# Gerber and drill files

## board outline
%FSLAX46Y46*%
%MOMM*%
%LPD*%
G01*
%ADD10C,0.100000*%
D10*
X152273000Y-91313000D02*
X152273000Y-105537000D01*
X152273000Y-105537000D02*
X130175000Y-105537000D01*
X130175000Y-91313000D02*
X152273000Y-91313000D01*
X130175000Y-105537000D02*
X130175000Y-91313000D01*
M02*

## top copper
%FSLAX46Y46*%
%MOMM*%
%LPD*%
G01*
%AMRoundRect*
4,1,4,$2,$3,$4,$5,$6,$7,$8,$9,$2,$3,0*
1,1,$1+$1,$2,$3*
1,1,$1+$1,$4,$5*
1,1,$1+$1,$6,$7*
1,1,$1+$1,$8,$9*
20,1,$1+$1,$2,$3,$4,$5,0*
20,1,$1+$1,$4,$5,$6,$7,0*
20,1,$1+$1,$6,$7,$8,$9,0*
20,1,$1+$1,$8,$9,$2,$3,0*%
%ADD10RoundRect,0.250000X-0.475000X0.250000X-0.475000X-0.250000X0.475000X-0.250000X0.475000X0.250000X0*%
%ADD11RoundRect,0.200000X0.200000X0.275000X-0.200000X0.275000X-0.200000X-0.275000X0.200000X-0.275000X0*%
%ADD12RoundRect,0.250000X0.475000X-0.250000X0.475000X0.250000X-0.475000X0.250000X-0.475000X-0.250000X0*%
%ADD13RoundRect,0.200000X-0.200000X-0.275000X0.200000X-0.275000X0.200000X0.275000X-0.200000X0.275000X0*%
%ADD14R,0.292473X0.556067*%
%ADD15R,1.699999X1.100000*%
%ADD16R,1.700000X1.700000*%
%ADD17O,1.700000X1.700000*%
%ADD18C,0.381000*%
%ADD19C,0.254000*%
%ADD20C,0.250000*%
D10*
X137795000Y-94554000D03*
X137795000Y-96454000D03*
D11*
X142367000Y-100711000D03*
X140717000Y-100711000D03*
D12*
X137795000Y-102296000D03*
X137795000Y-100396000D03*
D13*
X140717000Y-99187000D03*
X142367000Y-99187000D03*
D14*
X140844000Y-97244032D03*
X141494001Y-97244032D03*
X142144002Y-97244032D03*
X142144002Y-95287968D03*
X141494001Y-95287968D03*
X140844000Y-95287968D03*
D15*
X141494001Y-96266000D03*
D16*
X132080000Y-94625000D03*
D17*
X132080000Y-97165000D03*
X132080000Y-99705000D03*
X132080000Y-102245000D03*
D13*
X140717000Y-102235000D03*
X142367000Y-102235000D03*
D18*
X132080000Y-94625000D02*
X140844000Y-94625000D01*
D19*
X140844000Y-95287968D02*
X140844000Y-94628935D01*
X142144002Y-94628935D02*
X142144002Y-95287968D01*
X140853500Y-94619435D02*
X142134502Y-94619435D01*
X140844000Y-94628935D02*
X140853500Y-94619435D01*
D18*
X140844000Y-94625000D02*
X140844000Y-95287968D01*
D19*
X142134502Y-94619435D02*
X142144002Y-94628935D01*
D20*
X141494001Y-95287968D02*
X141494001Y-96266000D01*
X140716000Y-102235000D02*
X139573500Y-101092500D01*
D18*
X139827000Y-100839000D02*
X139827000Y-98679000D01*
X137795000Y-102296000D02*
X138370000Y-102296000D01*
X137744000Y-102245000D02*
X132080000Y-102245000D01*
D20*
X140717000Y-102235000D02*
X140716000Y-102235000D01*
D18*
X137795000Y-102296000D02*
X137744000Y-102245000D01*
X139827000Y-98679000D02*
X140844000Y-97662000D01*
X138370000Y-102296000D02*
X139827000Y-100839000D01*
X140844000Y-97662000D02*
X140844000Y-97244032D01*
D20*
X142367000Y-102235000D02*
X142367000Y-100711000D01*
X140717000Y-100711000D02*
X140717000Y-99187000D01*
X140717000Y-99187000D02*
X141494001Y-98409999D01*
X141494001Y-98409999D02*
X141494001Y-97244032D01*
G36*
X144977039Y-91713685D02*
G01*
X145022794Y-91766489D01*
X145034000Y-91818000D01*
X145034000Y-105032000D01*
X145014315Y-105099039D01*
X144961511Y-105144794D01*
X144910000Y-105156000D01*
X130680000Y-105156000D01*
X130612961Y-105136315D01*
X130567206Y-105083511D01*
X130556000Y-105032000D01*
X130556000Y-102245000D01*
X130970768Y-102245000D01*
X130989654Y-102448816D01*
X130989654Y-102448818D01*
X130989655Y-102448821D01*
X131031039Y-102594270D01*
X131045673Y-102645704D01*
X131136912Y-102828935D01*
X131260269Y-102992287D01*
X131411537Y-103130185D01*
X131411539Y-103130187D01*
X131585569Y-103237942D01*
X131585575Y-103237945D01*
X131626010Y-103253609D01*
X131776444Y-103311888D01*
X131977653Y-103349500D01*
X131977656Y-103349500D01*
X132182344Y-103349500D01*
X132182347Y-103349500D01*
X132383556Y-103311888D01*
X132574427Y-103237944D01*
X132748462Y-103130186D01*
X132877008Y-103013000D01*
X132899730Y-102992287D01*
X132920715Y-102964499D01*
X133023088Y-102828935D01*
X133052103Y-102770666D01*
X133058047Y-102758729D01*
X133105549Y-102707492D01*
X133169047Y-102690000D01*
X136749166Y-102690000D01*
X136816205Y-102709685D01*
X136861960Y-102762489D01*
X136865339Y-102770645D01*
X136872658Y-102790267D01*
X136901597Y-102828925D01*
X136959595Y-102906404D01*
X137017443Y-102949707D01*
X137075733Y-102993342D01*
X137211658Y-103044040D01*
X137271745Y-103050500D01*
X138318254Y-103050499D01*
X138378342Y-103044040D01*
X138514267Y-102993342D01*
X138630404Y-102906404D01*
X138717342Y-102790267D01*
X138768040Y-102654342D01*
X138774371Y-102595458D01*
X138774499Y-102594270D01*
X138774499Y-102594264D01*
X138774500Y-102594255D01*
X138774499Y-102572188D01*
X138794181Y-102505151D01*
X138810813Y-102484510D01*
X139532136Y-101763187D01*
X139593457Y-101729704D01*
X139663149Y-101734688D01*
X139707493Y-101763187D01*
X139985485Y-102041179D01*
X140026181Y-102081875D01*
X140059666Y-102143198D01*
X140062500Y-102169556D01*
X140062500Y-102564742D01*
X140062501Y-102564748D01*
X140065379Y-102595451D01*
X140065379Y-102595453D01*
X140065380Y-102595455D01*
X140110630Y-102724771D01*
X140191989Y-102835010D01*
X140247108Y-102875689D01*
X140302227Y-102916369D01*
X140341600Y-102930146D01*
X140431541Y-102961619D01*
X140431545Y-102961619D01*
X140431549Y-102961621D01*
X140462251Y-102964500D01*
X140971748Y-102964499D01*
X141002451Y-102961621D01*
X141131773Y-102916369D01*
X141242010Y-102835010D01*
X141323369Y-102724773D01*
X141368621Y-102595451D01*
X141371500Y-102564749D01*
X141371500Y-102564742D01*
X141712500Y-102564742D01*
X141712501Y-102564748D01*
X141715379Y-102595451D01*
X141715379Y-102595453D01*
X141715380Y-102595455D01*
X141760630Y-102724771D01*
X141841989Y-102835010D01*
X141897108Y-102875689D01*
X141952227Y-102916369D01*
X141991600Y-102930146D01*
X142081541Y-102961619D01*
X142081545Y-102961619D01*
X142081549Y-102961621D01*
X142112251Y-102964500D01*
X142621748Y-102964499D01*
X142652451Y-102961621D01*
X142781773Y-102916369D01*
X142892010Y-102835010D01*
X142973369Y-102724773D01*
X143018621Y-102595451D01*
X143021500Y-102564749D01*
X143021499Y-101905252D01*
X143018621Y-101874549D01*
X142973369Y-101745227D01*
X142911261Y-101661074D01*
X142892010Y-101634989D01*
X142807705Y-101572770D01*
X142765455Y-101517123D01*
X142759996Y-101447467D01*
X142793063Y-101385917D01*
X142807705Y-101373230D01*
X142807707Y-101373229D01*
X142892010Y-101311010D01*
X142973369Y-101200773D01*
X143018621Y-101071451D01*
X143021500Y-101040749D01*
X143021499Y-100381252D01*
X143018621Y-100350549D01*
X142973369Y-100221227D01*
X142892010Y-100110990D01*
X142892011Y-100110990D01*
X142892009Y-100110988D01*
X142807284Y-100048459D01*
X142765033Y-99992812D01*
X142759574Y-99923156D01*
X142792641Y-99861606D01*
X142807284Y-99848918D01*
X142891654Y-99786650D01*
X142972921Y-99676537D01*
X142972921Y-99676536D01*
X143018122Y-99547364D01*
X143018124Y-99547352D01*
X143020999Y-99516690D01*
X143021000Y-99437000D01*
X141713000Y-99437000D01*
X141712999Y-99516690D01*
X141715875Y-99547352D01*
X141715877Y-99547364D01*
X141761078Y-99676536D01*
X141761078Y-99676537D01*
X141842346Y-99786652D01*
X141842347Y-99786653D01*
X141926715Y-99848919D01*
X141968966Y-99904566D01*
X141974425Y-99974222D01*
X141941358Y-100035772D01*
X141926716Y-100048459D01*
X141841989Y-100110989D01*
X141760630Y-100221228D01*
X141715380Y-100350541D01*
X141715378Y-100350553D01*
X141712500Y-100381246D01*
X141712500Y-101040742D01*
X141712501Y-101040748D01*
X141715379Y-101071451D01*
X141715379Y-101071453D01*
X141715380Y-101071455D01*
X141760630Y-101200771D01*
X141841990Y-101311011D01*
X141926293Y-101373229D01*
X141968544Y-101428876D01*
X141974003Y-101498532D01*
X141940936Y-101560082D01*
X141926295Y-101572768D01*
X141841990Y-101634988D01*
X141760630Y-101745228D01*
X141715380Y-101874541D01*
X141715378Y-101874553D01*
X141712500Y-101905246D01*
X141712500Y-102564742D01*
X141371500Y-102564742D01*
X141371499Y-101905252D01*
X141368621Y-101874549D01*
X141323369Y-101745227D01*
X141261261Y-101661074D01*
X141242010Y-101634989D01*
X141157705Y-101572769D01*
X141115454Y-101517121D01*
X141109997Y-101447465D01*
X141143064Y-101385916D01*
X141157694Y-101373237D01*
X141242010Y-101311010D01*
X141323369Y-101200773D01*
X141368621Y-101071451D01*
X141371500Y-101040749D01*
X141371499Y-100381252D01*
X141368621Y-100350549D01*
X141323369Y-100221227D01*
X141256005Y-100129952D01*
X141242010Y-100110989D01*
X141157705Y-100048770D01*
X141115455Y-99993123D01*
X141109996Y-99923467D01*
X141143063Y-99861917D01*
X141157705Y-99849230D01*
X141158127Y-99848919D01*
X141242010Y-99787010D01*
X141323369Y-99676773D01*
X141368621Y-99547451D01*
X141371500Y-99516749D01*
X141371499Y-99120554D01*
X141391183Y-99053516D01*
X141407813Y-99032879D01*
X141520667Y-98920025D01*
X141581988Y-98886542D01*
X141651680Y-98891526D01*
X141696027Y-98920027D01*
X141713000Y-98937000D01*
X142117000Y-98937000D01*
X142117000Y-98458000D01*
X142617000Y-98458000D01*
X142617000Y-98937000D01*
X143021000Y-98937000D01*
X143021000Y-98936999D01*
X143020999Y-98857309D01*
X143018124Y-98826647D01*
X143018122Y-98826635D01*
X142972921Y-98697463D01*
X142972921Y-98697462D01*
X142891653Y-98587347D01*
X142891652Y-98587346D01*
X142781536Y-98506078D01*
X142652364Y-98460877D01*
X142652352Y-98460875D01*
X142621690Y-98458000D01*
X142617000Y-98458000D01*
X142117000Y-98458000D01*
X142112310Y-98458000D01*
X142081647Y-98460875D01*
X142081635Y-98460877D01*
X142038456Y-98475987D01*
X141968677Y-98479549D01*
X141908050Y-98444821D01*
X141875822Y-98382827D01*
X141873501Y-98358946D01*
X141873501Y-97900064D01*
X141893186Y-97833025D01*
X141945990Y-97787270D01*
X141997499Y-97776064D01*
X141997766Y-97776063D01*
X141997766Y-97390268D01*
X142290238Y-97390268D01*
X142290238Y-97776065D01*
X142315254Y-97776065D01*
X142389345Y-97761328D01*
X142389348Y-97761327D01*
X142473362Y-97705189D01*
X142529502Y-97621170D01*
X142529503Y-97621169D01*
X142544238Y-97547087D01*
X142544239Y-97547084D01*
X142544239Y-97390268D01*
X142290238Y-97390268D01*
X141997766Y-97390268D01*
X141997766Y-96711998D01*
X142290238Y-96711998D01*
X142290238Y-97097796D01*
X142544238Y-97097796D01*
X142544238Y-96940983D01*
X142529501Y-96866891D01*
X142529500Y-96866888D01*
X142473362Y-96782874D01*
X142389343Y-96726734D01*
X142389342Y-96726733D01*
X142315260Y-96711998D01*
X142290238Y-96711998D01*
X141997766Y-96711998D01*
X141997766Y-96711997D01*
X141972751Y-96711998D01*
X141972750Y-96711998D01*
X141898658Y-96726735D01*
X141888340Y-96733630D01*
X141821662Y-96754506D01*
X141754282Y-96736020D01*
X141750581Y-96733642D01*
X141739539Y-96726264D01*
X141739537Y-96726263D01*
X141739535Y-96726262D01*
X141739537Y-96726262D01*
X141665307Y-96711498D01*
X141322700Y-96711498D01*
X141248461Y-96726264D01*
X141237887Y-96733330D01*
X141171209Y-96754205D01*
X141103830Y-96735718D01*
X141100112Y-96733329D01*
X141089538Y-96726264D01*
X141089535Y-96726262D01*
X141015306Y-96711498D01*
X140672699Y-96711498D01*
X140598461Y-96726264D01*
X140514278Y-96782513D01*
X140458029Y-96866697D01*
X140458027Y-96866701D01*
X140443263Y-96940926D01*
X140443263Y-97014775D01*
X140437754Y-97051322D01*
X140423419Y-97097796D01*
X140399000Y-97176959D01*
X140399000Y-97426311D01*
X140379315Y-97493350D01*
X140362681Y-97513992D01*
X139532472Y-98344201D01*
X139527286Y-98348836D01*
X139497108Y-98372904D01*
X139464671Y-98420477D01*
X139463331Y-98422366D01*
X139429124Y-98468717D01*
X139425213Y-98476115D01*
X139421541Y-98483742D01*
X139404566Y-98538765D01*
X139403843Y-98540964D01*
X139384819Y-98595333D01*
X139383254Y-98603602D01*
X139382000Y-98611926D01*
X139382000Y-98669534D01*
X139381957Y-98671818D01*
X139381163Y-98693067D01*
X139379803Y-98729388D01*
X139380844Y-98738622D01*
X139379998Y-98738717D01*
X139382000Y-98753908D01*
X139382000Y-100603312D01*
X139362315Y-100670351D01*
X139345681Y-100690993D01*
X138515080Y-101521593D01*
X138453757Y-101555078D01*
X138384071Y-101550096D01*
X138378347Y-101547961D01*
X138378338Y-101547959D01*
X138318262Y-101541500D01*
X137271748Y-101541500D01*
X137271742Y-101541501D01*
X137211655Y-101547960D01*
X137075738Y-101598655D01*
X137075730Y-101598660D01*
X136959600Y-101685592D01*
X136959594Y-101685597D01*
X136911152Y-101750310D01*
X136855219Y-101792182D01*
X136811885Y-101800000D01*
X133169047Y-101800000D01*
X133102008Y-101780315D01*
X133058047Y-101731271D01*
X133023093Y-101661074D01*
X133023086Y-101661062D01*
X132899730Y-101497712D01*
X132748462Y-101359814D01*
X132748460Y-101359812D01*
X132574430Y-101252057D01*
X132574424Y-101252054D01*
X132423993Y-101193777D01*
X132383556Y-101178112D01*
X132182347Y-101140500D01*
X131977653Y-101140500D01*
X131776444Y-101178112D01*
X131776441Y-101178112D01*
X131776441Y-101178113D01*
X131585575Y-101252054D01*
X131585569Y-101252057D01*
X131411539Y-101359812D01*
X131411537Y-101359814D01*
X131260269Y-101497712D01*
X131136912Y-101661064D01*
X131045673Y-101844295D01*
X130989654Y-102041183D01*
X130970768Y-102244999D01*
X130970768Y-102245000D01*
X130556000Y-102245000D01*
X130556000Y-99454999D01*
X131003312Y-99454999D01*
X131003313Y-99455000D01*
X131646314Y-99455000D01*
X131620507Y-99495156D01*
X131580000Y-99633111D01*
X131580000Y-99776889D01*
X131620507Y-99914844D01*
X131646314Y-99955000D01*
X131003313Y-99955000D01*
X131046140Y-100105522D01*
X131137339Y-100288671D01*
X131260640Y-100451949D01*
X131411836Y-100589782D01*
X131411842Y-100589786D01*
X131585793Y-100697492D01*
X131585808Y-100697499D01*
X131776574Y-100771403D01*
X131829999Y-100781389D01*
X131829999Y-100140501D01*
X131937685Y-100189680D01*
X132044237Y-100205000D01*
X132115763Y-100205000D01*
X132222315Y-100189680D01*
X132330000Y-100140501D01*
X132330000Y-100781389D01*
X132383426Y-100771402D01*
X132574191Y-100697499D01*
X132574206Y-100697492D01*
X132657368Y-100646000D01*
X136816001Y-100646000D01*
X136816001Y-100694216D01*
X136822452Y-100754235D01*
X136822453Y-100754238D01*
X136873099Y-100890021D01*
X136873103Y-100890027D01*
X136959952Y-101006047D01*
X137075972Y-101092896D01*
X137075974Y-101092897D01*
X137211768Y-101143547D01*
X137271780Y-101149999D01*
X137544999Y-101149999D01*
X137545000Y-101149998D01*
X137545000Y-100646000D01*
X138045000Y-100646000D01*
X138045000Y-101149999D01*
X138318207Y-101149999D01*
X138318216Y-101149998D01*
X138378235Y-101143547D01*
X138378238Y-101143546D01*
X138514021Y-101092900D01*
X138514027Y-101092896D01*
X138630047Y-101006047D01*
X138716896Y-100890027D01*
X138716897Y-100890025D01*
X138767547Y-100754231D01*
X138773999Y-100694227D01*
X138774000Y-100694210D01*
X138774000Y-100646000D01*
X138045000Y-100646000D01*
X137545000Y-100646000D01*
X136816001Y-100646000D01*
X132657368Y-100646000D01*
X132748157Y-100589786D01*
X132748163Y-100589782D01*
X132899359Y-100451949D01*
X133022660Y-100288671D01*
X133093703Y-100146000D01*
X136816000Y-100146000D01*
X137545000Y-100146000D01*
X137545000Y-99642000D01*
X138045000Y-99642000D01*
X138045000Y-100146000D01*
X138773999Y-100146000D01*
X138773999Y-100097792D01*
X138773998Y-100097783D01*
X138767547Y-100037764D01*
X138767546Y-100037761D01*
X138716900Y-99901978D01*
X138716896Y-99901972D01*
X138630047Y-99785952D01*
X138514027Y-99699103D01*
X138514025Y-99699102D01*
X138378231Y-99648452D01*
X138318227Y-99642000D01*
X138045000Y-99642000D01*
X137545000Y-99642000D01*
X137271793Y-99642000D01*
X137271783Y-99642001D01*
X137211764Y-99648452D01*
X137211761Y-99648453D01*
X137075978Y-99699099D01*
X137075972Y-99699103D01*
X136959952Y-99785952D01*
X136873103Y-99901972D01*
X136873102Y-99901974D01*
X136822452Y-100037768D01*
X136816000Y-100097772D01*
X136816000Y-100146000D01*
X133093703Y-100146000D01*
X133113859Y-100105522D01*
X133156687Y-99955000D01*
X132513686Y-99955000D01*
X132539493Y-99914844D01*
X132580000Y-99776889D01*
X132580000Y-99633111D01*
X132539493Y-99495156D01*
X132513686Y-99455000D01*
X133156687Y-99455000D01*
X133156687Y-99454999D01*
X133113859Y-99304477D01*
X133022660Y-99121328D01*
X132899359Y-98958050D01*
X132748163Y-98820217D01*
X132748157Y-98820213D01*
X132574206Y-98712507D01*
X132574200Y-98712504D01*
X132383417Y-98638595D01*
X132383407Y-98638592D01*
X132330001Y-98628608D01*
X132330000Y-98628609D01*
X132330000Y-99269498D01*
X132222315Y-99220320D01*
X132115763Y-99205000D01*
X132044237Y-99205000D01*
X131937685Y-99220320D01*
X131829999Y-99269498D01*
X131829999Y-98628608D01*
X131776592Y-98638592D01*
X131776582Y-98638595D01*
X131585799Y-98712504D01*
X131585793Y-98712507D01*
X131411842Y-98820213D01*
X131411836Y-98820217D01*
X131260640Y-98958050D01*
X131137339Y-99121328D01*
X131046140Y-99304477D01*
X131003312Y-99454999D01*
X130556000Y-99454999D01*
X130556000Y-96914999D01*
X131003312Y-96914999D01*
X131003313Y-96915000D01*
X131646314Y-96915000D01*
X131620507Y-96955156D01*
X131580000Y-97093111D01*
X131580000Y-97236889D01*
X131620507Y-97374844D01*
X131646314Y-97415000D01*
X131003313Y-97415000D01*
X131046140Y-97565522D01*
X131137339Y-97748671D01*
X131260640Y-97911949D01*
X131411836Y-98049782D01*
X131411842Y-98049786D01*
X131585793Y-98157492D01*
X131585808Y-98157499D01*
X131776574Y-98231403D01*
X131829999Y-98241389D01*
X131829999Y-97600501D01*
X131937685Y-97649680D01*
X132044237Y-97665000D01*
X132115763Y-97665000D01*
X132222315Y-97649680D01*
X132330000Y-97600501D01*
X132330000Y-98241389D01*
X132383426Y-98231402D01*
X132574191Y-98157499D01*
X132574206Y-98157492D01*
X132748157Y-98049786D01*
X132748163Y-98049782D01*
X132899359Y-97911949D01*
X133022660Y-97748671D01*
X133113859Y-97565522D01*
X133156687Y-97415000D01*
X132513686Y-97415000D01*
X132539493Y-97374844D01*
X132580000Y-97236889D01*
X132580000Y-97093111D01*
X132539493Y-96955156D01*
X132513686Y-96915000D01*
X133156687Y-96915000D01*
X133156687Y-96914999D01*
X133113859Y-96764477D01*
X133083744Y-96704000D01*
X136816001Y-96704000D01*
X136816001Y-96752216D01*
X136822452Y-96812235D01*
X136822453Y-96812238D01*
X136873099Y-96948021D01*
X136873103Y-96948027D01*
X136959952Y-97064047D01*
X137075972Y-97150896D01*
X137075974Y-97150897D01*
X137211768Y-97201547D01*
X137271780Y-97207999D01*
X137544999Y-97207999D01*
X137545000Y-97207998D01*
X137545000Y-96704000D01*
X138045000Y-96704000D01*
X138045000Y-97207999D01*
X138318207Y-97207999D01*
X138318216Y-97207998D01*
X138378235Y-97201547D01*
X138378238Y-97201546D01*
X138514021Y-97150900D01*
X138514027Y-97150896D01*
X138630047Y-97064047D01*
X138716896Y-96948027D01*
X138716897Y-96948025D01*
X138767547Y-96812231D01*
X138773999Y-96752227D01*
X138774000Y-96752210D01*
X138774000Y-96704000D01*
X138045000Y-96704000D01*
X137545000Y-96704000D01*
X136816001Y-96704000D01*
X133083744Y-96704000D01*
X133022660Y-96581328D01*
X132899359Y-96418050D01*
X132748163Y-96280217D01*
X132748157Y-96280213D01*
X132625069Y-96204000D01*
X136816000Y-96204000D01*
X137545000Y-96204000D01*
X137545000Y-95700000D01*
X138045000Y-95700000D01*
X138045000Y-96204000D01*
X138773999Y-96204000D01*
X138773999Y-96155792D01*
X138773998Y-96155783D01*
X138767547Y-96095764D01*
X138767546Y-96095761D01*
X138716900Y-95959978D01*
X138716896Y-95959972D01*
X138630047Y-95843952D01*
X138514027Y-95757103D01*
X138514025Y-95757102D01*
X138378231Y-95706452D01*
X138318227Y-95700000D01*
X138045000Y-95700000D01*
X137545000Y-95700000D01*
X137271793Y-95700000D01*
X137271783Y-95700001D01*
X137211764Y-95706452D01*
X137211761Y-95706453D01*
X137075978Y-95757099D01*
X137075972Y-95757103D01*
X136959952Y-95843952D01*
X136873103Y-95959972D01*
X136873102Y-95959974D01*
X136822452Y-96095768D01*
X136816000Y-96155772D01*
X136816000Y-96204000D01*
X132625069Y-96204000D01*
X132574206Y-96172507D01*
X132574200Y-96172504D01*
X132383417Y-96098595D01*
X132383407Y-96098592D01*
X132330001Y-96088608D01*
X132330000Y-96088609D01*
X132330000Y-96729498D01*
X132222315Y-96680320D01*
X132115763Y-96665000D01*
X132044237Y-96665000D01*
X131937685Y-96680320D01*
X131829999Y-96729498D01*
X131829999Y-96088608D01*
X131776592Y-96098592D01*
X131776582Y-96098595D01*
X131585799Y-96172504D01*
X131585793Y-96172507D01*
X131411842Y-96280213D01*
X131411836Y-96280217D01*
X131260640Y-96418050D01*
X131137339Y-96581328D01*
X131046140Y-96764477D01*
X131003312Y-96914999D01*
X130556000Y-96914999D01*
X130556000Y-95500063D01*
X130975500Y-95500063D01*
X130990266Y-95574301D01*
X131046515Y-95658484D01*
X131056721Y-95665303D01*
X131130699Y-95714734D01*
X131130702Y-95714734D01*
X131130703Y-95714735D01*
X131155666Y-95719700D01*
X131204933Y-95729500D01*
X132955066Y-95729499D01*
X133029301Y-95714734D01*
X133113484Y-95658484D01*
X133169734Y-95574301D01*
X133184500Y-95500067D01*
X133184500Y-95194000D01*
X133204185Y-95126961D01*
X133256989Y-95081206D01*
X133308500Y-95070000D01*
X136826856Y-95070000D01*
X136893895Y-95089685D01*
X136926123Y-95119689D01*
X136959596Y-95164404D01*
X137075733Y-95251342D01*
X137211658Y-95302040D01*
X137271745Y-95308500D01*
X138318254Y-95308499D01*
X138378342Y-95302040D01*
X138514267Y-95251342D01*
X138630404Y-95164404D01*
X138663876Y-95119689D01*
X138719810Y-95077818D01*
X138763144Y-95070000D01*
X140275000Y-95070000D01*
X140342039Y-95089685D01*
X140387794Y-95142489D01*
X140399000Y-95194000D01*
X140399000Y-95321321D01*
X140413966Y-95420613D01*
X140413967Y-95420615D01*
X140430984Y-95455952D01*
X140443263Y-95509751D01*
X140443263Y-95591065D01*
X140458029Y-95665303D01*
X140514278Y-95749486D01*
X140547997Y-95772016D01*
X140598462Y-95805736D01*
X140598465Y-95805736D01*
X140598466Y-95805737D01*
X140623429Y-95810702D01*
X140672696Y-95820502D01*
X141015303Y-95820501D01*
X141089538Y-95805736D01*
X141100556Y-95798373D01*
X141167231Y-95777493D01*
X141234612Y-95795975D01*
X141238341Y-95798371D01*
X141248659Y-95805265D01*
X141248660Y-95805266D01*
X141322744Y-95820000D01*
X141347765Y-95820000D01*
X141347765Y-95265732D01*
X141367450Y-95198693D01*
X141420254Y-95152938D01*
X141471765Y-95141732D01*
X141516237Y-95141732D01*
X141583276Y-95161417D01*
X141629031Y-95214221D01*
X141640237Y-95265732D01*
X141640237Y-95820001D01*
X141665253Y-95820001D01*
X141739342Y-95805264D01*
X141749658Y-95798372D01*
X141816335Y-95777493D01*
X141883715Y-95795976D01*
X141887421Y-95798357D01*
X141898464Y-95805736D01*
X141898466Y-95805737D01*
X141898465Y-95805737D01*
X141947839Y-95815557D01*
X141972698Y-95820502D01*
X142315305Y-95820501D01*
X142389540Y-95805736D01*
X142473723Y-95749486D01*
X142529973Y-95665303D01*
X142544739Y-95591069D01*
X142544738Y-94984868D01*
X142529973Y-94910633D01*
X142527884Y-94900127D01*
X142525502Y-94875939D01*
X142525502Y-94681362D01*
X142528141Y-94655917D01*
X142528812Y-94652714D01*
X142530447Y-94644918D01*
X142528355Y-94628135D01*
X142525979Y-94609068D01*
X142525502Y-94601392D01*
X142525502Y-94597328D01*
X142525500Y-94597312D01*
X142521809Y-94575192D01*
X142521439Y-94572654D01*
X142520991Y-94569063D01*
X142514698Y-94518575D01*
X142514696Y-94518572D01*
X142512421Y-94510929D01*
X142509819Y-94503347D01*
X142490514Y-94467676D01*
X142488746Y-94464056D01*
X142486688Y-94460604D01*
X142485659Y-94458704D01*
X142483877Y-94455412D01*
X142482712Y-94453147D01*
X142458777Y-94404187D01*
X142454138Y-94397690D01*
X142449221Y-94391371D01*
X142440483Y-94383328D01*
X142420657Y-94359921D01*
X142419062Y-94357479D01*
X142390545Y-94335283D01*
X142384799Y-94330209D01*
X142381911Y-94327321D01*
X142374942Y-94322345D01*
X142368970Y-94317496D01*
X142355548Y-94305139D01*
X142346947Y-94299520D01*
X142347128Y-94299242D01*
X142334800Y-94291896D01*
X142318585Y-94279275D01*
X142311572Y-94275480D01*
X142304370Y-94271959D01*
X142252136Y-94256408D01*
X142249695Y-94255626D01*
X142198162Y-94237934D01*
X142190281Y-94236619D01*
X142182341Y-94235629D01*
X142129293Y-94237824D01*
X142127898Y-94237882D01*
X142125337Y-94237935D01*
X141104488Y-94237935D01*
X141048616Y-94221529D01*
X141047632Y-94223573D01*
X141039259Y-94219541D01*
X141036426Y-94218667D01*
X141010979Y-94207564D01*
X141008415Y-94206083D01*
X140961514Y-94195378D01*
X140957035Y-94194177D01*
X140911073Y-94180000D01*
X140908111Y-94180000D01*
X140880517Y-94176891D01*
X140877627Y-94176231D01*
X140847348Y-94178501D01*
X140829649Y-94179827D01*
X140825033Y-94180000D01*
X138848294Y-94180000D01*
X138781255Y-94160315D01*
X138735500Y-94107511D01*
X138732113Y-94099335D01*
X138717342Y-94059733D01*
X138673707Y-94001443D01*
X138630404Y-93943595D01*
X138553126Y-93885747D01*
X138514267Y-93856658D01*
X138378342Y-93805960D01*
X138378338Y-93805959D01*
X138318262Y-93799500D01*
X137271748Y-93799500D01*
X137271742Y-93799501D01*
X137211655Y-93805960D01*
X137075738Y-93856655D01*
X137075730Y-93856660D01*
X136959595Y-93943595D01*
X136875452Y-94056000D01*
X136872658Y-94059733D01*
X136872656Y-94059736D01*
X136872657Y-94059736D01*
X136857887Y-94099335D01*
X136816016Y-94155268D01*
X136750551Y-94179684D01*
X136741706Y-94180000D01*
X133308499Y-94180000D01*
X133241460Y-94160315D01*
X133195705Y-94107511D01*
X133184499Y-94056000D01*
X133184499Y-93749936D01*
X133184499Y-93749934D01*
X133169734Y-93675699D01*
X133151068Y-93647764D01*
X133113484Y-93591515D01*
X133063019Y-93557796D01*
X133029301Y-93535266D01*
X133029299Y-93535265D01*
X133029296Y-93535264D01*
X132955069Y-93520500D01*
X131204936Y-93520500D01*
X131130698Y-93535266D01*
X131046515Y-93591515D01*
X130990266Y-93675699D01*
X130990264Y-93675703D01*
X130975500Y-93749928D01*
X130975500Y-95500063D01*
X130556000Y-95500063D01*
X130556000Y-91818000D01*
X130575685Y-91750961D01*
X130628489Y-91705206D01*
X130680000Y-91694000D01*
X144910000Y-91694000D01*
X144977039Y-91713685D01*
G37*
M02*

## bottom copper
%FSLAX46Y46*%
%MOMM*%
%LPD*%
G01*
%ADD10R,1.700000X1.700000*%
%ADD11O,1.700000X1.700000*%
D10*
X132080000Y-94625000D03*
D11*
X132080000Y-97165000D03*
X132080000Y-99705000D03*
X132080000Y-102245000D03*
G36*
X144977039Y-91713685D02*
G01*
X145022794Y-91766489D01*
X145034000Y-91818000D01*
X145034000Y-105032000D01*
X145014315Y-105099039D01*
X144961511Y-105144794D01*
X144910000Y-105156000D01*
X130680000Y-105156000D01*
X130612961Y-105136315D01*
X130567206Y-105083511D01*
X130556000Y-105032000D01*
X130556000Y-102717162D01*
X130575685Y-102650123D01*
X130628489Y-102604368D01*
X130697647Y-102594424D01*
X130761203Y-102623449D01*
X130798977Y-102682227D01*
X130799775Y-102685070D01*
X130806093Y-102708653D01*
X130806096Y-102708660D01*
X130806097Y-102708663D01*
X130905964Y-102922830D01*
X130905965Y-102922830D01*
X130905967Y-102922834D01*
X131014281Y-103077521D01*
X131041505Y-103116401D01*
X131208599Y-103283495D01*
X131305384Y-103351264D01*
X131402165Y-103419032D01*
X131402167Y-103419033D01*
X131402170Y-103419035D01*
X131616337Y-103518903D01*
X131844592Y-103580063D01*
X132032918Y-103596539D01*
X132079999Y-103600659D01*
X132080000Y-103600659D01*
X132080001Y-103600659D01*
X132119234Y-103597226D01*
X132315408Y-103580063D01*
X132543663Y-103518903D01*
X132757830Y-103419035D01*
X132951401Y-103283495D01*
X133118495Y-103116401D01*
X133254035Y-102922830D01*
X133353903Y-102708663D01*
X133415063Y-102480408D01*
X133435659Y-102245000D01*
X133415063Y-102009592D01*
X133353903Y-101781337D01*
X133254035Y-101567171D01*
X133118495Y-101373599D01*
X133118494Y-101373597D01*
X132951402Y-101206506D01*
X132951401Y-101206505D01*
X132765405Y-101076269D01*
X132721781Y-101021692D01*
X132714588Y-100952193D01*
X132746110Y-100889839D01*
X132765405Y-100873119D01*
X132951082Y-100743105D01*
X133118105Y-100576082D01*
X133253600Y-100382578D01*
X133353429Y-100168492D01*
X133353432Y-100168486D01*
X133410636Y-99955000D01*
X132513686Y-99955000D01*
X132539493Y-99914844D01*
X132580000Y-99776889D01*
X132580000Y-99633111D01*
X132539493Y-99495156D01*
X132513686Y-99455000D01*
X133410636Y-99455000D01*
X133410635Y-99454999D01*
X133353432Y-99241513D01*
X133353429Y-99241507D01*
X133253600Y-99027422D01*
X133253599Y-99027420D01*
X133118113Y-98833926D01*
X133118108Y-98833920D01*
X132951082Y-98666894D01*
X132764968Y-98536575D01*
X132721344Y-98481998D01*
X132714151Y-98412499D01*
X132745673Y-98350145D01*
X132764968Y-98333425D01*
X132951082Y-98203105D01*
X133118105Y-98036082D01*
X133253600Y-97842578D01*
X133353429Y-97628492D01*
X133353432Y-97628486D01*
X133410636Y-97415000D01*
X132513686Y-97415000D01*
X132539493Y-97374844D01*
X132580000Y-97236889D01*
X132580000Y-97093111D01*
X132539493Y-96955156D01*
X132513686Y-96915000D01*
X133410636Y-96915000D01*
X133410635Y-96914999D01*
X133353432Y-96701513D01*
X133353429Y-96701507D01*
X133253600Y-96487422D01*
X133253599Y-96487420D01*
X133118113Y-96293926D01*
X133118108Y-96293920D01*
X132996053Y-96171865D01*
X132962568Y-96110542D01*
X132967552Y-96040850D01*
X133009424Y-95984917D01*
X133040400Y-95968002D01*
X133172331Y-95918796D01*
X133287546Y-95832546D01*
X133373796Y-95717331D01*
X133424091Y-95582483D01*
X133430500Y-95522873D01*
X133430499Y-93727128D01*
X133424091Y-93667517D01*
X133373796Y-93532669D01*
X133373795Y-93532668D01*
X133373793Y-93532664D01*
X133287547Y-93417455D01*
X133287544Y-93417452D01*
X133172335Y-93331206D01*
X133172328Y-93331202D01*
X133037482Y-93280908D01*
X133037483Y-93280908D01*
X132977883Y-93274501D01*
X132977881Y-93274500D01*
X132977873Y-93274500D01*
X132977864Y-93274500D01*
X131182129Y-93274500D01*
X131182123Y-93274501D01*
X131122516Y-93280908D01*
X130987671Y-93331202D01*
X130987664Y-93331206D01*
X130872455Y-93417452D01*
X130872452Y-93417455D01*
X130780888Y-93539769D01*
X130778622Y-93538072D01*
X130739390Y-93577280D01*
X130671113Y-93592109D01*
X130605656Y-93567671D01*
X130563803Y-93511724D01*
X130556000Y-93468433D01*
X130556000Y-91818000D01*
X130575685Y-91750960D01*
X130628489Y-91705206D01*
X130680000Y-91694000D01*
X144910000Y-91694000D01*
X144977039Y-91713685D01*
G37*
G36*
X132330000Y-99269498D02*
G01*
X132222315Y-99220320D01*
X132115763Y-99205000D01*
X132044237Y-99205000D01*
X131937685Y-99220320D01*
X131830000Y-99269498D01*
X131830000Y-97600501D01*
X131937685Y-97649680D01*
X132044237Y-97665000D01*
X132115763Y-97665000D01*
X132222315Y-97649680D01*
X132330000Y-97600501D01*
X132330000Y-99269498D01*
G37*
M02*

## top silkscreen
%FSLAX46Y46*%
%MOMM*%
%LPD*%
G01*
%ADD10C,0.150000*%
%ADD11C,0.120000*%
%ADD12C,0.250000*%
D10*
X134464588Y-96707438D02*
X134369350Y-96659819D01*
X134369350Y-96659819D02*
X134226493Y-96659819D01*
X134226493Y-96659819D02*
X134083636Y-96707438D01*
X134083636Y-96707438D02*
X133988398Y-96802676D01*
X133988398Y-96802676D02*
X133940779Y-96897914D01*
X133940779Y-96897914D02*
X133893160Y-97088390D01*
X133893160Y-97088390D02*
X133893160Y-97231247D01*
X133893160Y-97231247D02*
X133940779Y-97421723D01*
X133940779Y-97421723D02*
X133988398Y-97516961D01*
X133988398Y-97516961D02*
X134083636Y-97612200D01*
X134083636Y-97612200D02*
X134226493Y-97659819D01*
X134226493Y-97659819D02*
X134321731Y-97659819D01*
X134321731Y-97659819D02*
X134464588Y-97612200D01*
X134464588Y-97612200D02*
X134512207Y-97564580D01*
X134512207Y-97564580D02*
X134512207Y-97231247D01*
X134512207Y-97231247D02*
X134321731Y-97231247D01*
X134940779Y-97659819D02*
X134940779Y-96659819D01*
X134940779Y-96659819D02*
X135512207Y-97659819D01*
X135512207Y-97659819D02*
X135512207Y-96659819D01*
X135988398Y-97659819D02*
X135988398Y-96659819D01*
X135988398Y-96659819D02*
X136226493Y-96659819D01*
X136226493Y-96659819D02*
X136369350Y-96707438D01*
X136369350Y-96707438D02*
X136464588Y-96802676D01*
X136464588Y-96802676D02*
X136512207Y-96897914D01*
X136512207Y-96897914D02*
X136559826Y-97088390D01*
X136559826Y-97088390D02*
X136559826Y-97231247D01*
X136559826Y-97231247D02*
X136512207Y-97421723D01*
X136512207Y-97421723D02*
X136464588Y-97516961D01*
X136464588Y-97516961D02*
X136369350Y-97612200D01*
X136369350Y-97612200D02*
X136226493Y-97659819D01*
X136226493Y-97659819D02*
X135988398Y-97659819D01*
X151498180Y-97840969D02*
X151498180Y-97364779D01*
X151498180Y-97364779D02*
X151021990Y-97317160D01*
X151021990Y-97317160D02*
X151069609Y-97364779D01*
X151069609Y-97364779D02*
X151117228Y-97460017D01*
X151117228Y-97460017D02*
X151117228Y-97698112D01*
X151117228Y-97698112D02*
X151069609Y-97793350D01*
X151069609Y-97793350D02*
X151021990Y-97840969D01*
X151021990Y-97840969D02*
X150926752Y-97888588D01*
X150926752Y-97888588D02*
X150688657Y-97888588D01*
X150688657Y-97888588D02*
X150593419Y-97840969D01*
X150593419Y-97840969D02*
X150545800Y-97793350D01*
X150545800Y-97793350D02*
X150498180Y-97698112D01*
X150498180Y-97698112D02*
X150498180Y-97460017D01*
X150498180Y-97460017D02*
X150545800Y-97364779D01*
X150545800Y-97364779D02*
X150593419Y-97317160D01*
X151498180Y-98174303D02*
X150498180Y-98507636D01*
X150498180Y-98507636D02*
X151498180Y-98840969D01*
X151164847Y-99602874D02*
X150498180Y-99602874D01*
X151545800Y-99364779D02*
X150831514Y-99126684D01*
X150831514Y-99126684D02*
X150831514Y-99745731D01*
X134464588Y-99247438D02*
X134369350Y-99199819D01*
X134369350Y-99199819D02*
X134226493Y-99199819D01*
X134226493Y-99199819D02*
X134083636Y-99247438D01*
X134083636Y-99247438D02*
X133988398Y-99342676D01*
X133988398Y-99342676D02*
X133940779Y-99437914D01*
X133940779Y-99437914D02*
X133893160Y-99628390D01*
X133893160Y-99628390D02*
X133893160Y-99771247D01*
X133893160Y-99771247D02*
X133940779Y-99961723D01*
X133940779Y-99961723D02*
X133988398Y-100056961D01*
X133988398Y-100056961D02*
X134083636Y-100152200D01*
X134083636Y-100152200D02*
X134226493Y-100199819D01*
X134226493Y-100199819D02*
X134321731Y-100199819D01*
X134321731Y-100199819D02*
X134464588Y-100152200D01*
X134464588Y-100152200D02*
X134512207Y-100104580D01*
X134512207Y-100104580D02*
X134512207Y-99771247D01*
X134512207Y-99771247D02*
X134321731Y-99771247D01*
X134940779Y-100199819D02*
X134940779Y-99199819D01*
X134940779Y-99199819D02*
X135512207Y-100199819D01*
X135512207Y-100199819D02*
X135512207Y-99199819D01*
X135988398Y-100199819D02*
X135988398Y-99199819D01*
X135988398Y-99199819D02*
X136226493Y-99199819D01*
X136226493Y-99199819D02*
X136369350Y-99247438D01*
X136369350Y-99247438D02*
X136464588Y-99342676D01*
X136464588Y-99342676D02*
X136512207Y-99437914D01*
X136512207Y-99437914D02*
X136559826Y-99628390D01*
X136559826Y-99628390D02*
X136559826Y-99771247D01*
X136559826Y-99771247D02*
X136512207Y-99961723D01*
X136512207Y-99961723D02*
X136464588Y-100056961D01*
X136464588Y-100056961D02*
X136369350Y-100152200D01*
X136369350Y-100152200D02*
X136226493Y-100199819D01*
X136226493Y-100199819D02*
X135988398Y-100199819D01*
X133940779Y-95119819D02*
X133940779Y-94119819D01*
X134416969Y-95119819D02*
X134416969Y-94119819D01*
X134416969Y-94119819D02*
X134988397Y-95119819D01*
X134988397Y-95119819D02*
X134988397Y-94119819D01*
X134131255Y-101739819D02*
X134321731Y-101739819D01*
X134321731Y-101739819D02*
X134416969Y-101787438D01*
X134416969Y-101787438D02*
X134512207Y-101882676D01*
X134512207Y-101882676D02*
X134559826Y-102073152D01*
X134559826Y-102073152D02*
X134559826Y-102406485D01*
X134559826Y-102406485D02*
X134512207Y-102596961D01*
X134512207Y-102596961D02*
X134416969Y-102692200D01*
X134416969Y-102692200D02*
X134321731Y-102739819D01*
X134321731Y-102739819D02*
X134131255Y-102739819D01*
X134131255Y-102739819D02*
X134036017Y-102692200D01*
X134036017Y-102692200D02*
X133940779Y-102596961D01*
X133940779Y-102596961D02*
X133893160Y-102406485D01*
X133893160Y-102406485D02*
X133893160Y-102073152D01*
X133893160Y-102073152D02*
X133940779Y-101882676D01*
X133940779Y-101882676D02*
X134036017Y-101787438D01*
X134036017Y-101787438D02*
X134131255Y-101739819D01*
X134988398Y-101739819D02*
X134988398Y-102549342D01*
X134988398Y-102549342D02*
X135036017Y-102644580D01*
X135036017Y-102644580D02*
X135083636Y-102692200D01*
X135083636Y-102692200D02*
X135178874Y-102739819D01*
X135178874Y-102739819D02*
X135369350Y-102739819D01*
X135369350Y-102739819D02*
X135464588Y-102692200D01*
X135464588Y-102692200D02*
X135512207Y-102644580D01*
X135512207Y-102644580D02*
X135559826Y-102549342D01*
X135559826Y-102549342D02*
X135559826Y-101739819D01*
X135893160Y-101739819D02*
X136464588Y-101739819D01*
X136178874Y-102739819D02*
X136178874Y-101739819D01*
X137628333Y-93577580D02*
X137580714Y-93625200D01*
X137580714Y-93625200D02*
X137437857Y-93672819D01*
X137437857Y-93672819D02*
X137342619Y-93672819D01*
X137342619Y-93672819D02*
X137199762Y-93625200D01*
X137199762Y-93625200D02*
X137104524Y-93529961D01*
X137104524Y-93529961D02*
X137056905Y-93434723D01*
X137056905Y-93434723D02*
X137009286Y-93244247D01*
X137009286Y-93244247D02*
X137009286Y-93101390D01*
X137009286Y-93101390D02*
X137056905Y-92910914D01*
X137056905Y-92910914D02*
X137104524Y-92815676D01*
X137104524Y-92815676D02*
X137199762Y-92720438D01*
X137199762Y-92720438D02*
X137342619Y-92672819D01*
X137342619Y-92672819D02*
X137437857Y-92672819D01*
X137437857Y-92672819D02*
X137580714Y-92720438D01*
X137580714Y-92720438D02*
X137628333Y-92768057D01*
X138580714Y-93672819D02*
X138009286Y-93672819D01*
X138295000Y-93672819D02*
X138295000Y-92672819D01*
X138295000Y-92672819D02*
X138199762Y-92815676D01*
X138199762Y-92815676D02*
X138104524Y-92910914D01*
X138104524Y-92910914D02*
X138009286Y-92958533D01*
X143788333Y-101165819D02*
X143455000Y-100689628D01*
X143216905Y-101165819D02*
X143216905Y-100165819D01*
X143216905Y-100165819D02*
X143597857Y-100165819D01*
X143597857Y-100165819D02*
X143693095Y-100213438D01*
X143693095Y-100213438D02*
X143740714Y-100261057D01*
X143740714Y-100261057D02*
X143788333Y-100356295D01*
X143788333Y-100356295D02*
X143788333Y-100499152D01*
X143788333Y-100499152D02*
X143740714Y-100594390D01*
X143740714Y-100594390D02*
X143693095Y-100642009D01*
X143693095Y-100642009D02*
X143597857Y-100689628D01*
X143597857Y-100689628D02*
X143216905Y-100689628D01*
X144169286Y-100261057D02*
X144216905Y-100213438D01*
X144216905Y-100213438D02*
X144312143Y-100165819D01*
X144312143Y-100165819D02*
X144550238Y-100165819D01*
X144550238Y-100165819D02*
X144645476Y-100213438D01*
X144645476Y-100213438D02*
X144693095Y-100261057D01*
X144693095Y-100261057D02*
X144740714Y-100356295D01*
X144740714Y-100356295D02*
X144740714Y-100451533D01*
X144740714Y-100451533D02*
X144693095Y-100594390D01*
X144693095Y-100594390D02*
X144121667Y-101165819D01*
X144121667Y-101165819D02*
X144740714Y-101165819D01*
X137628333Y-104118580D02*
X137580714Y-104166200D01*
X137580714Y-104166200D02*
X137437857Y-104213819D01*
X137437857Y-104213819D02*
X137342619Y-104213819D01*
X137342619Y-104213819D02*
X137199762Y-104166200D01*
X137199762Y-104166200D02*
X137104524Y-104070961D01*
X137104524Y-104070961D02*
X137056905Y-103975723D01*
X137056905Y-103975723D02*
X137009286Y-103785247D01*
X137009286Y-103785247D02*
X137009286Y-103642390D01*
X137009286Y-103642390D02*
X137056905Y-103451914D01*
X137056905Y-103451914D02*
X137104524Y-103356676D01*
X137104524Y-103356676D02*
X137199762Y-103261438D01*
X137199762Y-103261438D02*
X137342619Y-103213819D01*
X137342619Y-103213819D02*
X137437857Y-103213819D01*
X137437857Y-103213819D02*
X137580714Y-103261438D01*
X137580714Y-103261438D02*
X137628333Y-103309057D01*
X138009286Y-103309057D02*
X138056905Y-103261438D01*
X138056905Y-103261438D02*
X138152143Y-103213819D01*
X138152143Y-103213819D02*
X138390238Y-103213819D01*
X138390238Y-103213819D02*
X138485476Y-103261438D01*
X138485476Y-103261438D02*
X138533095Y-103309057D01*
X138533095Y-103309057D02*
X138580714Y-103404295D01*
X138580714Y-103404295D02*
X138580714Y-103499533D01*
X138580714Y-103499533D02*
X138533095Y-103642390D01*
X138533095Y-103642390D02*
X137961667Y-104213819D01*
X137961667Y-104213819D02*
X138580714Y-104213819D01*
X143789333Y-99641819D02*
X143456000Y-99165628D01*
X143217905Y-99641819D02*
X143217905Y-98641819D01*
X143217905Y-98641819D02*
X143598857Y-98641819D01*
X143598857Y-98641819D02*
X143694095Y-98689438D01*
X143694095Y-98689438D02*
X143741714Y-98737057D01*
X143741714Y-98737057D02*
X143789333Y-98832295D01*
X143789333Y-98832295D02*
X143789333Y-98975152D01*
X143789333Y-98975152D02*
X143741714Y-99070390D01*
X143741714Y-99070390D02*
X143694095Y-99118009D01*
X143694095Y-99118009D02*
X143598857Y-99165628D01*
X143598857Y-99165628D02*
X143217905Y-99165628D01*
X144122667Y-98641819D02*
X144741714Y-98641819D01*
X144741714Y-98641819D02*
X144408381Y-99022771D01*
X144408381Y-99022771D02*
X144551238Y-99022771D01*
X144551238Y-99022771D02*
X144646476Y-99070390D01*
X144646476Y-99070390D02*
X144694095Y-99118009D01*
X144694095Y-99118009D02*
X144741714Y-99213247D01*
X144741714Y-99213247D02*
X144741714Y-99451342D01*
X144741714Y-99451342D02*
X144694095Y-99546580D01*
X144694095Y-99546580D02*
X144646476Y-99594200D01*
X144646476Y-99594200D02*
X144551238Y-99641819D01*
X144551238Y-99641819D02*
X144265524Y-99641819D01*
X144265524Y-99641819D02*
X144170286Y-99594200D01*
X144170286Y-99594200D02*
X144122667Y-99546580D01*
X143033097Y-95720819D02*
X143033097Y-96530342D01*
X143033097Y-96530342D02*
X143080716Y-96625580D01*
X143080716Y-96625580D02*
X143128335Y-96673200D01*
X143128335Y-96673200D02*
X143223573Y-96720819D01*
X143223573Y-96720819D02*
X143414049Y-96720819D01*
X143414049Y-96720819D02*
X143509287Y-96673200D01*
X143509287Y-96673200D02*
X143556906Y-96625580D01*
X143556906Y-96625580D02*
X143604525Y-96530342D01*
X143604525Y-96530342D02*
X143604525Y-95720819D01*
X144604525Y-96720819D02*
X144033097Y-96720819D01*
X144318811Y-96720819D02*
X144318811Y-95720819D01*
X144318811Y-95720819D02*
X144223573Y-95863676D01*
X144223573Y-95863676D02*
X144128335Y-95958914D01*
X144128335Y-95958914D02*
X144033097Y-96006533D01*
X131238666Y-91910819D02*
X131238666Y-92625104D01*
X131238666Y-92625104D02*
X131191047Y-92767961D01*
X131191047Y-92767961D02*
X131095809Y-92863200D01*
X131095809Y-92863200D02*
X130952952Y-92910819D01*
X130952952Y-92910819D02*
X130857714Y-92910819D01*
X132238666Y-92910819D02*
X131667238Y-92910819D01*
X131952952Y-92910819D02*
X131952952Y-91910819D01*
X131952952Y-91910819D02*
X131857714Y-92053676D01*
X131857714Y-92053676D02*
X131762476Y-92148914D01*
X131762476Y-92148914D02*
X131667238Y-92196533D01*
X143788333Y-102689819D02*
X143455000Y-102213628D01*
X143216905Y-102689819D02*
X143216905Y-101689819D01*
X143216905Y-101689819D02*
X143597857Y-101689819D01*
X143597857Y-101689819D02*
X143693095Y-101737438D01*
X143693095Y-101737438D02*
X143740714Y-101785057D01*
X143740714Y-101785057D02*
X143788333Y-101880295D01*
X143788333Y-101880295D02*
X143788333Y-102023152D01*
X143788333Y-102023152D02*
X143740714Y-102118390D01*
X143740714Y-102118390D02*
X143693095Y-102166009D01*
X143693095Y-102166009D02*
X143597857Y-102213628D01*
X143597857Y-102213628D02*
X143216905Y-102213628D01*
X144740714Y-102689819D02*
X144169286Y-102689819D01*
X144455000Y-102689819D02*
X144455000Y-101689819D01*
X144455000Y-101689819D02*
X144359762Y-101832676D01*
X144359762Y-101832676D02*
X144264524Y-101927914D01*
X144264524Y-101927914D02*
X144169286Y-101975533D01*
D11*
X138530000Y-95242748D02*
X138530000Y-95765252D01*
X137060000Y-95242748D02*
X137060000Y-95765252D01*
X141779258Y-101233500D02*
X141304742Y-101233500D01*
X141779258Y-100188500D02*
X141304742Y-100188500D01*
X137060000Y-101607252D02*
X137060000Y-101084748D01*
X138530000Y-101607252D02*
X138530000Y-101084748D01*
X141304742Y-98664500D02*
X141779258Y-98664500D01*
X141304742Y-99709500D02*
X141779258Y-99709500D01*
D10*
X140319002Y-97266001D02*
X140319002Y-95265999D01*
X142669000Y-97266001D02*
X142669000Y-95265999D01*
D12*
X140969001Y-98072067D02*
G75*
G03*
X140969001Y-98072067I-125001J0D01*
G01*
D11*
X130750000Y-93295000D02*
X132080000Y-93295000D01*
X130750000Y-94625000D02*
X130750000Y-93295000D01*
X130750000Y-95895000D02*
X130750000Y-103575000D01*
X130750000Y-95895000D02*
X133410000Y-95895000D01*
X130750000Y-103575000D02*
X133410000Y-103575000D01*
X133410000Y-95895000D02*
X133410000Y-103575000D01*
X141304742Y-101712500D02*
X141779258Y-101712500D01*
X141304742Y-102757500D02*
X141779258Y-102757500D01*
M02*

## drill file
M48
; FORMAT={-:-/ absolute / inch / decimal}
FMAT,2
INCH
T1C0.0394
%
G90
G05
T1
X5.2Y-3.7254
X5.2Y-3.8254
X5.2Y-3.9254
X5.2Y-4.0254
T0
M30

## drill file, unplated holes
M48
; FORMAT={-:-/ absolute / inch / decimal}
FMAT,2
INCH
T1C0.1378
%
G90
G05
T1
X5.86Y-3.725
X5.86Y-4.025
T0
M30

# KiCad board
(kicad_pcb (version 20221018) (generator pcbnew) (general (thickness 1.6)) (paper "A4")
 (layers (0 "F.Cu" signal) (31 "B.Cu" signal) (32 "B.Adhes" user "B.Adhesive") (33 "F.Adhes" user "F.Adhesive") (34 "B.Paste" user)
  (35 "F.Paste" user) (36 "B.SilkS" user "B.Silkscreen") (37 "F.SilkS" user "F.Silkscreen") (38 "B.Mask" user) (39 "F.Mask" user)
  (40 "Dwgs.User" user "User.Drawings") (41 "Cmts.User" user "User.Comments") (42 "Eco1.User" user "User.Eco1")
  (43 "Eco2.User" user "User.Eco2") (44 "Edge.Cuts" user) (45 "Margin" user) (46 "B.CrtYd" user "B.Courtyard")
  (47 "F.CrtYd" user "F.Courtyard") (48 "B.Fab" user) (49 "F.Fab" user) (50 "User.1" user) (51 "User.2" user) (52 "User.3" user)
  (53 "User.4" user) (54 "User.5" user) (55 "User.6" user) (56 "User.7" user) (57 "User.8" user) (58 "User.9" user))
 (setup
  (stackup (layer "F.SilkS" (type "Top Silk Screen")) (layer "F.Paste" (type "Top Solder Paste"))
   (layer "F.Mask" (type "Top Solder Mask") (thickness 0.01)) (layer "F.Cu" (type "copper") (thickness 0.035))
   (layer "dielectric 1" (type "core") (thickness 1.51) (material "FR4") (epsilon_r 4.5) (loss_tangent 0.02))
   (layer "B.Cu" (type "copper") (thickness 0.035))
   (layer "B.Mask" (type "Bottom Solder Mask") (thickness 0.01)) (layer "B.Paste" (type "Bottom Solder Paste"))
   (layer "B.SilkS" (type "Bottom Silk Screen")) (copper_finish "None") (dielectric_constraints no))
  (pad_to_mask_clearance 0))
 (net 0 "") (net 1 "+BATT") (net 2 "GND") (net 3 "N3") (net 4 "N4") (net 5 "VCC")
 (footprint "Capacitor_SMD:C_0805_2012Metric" (layer "F.Cu") (at 137.795 95.504 -90)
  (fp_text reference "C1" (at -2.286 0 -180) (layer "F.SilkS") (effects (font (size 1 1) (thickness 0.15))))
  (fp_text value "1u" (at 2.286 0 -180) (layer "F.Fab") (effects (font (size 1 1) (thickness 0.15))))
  (fp_line (start -0.261252 -0.735) (end 0.261252 -0.735) (stroke (width 0.12) (type solid)) (layer "F.SilkS"))
  (fp_line (start -0.261252 0.735) (end 0.261252 0.735) (stroke (width 0.12) (type solid)) (layer "F.SilkS"))
  (pad "1" smd roundrect (at -0.95 0 270) (size 1 1.45) (layers "F.Cu" "F.Paste" "F.Mask") (roundrect_rratio 0.25) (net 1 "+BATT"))
  (pad "2" smd roundrect (at 0.95 0 270) (size 1 1.45) (layers "F.Cu" "F.Paste" "F.Mask") (roundrect_rratio 0.25) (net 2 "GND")))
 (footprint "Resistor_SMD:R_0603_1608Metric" (layer "F.Cu") (at 141.542 100.711 180)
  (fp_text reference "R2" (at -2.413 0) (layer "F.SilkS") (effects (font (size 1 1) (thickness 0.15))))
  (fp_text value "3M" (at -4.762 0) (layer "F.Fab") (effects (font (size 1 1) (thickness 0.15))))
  (fp_line (start -0.237258 -0.5225) (end 0.237258 -0.5225) (stroke (width 0.12) (type solid)) (layer "F.SilkS"))
  (fp_line (start -0.237258 0.5225) (end 0.237258 0.5225) (stroke (width 0.12) (type solid)) (layer "F.SilkS"))
  (pad "1" smd roundrect (at -0.825 0 180) (size 0.8 0.95) (layers "F.Cu" "F.Paste" "F.Mask") (roundrect_rratio 0.25) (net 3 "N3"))
  (pad "2" smd roundrect (at 0.825 0 180) (size 0.8 0.95) (layers "F.Cu" "F.Paste" "F.Mask") (roundrect_rratio 0.25) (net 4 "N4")))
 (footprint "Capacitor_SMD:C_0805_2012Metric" (layer "F.Cu") (at 137.795 101.346 90)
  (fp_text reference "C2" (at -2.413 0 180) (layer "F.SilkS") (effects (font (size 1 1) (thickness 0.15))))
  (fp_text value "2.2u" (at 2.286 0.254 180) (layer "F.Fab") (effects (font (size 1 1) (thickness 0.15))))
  (fp_line (start -0.261252 -0.735) (end 0.261252 -0.735) (stroke (width 0.12) (type solid)) (layer "F.SilkS"))
  (fp_line (start -0.261252 0.735) (end 0.261252 0.735) (stroke (width 0.12) (type solid)) (layer "F.SilkS"))
  (pad "1" smd roundrect (at -0.95 0 90) (size 1 1.45) (layers "F.Cu" "F.Paste" "F.Mask") (roundrect_rratio 0.25) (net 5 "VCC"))
  (pad "2" smd roundrect (at 0.95 0 90) (size 1 1.45) (layers "F.Cu" "F.Paste" "F.Mask") (roundrect_rratio 0.25) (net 2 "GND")))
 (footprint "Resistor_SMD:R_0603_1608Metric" (layer "F.Cu") (at 141.542 99.187)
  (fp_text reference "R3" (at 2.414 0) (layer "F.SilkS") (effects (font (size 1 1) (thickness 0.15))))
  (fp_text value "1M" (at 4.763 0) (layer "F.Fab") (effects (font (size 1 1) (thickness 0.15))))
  (fp_line (start -0.237258 -0.5225) (end 0.237258 -0.5225) (stroke (width 0.12) (type solid)) (layer "F.SilkS"))
  (fp_line (start -0.237258 0.5225) (end 0.237258 0.5225) (stroke (width 0.12) (type solid)) (layer "F.SilkS"))
  (pad "1" smd roundrect (at -0.825 0) (size 0.8 0.95) (layers "F.Cu" "F.Paste" "F.Mask") (roundrect_rratio 0.25) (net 4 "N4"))
  (pad "2" smd roundrect (at 0.825 0) (size 0.8 0.95) (layers "F.Cu" "F.Paste" "F.Mask") (roundrect_rratio 0.25) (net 2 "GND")))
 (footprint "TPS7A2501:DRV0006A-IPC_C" (layer "F.Cu") (at 141.494001 96.266 90)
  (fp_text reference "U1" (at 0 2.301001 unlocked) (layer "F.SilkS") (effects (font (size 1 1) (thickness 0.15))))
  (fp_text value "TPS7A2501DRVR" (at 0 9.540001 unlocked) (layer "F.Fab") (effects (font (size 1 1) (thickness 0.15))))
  (fp_line (start -1.000001 -1.174999) (end 1.000001 -1.174999) (stroke (width 0.15) (type solid)) (layer "F.SilkS"))
  (fp_line (start -1.000001 1.174999) (end 1.000001 1.174999) (stroke (width 0.15) (type solid)) (layer "F.SilkS"))
  (fp_circle (center -1.806067 -0.650001) (end -1.681066 -0.650001) (stroke (width 0.25) (type solid)) (fill none) (layer "F.SilkS"))
  (pad "1" smd rect (at -0.978032 -0.650001 90) (size 0.556067 0.292473) (layers "F.Cu" "F.Paste" "F.Mask") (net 5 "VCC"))
  (pad "2" smd rect (at -0.978032 0 90) (size 0.556067 0.292473) (layers "F.Cu" "F.Paste" "F.Mask") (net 4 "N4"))
  (pad "3" smd rect (at -0.978032 0.650001 90) (size 0.556067 0.292473) (layers "F.Cu" "F.Paste" "F.Mask") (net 2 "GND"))
  (pad "4" smd rect (at 0.978032 0.650001 90) (size 0.556067 0.292473) (layers "F.Cu" "F.Paste" "F.Mask") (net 1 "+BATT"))
  (pad "5" smd rect (at 0.978032 0 90) (size 0.556067 0.292473) (layers "F.Cu" "F.Paste" "F.Mask") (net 2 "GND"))
  (pad "6" smd rect (at 0.978032 -0.650001 90) (size 0.556067 0.292473) (layers "F.Cu" "F.Paste" "F.Mask") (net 1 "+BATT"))
  (pad "7" smd rect (at 0 0 90) (size 1.1 1.699999) (layers "F.Cu" "F.Mask") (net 2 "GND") (zone_connect 2)))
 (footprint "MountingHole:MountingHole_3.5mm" (layer "F.Cu") (at 148.844 94.615)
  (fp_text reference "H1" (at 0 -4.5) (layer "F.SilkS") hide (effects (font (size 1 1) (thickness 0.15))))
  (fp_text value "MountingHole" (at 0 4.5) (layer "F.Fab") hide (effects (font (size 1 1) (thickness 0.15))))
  (pad "" np_thru_hole circle (at 0 0) (size 3.5 3.5) (drill 3.5) (layers "*.Cu" "*.Mask")))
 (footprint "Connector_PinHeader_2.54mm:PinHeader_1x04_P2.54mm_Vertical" (layer "F.Cu") (at 132.08 94.625)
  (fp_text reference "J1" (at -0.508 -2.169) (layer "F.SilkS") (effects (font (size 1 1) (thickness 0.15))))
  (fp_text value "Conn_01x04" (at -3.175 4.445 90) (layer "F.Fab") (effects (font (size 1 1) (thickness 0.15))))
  (fp_line (start -1.33 -1.33) (end 0 -1.33) (stroke (width 0.12) (type solid)) (layer "F.SilkS"))
  (fp_line (start -1.33 0) (end -1.33 -1.33) (stroke (width 0.12) (type solid)) (layer "F.SilkS"))
  (fp_line (start -1.33 1.27) (end -1.33 8.95) (stroke (width 0.12) (type solid)) (layer "F.SilkS"))
  (fp_line (start -1.33 1.27) (end 1.33 1.27) (stroke (width 0.12) (type solid)) (layer "F.SilkS"))
  (fp_line (start -1.33 8.95) (end 1.33 8.95) (stroke (width 0.12) (type solid)) (layer "F.SilkS"))
  (fp_line (start 1.33 1.27) (end 1.33 8.95) (stroke (width 0.12) (type solid)) (layer "F.SilkS"))
  (pad "1" thru_hole rect (at 0 0) (size 1.7 1.7) (drill 1) (layers "*.Cu" "*.Mask") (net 1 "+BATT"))
  (pad "2" thru_hole oval (at 0 2.54) (size 1.7 1.7) (drill 1) (layers "*.Cu" "*.Mask") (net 2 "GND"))
  (pad "3" thru_hole oval (at 0 5.08) (size 1.7 1.7) (drill 1) (layers "*.Cu" "*.Mask") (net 2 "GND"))
  (pad "4" thru_hole oval (at 0 7.62) (size 1.7 1.7) (drill 1) (layers "*.Cu" "*.Mask") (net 5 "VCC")))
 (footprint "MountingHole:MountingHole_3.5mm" (layer "F.Cu") (at 148.844 102.235)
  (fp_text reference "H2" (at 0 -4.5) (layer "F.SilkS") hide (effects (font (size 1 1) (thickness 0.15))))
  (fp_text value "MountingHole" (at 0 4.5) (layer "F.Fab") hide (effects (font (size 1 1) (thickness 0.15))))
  (pad "" np_thru_hole circle (at 0 0) (size 3.5 3.5) (drill 3.5) (layers "*.Cu" "*.Mask")))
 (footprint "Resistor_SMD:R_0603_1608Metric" (layer "F.Cu") (at 141.542 102.235)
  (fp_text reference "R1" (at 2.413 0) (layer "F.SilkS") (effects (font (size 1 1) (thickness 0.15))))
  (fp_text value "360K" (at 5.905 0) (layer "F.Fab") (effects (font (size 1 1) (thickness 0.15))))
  (fp_line (start -0.237258 -0.5225) (end 0.237258 -0.5225) (stroke (width 0.12) (type solid)) (layer "F.SilkS"))
  (fp_line (start -0.237258 0.5225) (end 0.237258 0.5225) (stroke (width 0.12) (type solid)) (layer "F.SilkS"))
  (pad "1" smd roundrect (at -0.825 0) (size 0.8 0.95) (layers "F.Cu" "F.Paste" "F.Mask") (roundrect_rratio 0.25) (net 5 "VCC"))
  (pad "2" smd roundrect (at 0.825 0) (size 0.8 0.95) (layers "F.Cu" "F.Paste" "F.Mask") (roundrect_rratio 0.25) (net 3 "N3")))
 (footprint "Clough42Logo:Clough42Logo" (layer "B.Cu") (at 139.954 98.679 -90)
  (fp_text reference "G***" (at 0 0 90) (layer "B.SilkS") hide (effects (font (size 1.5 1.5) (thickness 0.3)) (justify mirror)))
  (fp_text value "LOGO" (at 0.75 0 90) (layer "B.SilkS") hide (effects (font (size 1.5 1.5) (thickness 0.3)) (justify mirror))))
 (gr_line (start 152.273 91.313) (end 152.273 105.537) (stroke (width 0.1) (type default)) (layer "Edge.Cuts"))
 (gr_line (start 152.273 105.537) (end 130.175 105.537) (stroke (width 0.1) (type default)) (layer "Edge.Cuts"))
 (gr_line (start 130.175 91.313) (end 152.273 91.313) (stroke (width 0.1) (type default)) (layer "Edge.Cuts"))
 (gr_line (start 130.175 105.537) (end 130.175 91.313) (stroke (width 0.1) (type default)) (layer "Edge.Cuts"))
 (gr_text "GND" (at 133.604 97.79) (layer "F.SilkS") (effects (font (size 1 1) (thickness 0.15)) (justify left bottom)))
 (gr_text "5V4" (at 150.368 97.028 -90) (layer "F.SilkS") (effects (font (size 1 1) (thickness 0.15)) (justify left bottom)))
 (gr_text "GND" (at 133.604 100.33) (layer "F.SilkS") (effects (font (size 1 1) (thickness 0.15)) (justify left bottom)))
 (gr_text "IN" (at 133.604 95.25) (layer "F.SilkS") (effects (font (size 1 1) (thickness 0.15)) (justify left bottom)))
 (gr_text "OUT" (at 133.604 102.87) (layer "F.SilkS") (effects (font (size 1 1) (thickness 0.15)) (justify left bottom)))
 (segment (start 132.08 94.625) (end 140.844 94.625) (width 0.381) (layer "F.Cu") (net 1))
 (segment (start 140.844 95.287968) (end 140.844 94.628935) (width 0.254) (layer "F.Cu") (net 1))
 (segment (start 142.144002 94.628935) (end 142.144002 95.287968) (width 0.254) (layer "F.Cu") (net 1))
 (segment (start 140.8535 94.619435) (end 142.134502 94.619435) (width 0.254) (layer "F.Cu") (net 1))
 (segment (start 140.844 94.628935) (end 140.8535 94.619435) (width 0.254) (layer "F.Cu") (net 1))
 (segment (start 140.844 94.625) (end 140.844 95.287968) (width 0.381) (layer "F.Cu") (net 1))
 (segment (start 142.134502 94.619435) (end 142.144002 94.628935) (width 0.254) (layer "F.Cu") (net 1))
 (segment (start 141.494001 95.287968) (end 141.494001 96.266) (width 0.25) (layer "F.Cu") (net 2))
 (segment (start 140.716 102.235) (end 139.5735 101.0925) (width 0.25) (layer "F.Cu") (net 5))
 (segment (start 139.827 100.839) (end 139.827 98.679) (width 0.381) (layer "F.Cu") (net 5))
 (segment (start 137.795 102.296) (end 138.37 102.296) (width 0.381) (layer "F.Cu") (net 5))
 (segment (start 137.744 102.245) (end 132.08 102.245) (width 0.381) (layer "F.Cu") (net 5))
 (segment (start 140.717 102.235) (end 140.716 102.235) (width 0.25) (layer "F.Cu") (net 5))
 (segment (start 137.795 102.296) (end 137.744 102.245) (width 0.381) (layer "F.Cu") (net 5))
 (segment (start 139.827 98.679) (end 140.844 97.662) (width 0.381) (layer "F.Cu") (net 5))
 (segment (start 138.37 102.296) (end 139.827 100.839) (width 0.381) (layer "F.Cu") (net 5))
 (segment (start 140.844 97.662) (end 140.844 97.244032) (width 0.381) (layer "F.Cu") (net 5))
 (segment (start 142.367 102.235) (end 142.367 100.711) (width 0.25) (layer "F.Cu") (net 3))
 (segment (start 140.717 100.711) (end 140.717 99.187) (width 0.25) (layer "F.Cu") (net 4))
 (segment (start 140.717 99.187) (end 141.494001 98.409999) (width 0.25) (layer "F.Cu") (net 4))
 (segment (start 141.494001 98.409999) (end 141.494001 97.244032) (width 0.25) (layer "F.Cu") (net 4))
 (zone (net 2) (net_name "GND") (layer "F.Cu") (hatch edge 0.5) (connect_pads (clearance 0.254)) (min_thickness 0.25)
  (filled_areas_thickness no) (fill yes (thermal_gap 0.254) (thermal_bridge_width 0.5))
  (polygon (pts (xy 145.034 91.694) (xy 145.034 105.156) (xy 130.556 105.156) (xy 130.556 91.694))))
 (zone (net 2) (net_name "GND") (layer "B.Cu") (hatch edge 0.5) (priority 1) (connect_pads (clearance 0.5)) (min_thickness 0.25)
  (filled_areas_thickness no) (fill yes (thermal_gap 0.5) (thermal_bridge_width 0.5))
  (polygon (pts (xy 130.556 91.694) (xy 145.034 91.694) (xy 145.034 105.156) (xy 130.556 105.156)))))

